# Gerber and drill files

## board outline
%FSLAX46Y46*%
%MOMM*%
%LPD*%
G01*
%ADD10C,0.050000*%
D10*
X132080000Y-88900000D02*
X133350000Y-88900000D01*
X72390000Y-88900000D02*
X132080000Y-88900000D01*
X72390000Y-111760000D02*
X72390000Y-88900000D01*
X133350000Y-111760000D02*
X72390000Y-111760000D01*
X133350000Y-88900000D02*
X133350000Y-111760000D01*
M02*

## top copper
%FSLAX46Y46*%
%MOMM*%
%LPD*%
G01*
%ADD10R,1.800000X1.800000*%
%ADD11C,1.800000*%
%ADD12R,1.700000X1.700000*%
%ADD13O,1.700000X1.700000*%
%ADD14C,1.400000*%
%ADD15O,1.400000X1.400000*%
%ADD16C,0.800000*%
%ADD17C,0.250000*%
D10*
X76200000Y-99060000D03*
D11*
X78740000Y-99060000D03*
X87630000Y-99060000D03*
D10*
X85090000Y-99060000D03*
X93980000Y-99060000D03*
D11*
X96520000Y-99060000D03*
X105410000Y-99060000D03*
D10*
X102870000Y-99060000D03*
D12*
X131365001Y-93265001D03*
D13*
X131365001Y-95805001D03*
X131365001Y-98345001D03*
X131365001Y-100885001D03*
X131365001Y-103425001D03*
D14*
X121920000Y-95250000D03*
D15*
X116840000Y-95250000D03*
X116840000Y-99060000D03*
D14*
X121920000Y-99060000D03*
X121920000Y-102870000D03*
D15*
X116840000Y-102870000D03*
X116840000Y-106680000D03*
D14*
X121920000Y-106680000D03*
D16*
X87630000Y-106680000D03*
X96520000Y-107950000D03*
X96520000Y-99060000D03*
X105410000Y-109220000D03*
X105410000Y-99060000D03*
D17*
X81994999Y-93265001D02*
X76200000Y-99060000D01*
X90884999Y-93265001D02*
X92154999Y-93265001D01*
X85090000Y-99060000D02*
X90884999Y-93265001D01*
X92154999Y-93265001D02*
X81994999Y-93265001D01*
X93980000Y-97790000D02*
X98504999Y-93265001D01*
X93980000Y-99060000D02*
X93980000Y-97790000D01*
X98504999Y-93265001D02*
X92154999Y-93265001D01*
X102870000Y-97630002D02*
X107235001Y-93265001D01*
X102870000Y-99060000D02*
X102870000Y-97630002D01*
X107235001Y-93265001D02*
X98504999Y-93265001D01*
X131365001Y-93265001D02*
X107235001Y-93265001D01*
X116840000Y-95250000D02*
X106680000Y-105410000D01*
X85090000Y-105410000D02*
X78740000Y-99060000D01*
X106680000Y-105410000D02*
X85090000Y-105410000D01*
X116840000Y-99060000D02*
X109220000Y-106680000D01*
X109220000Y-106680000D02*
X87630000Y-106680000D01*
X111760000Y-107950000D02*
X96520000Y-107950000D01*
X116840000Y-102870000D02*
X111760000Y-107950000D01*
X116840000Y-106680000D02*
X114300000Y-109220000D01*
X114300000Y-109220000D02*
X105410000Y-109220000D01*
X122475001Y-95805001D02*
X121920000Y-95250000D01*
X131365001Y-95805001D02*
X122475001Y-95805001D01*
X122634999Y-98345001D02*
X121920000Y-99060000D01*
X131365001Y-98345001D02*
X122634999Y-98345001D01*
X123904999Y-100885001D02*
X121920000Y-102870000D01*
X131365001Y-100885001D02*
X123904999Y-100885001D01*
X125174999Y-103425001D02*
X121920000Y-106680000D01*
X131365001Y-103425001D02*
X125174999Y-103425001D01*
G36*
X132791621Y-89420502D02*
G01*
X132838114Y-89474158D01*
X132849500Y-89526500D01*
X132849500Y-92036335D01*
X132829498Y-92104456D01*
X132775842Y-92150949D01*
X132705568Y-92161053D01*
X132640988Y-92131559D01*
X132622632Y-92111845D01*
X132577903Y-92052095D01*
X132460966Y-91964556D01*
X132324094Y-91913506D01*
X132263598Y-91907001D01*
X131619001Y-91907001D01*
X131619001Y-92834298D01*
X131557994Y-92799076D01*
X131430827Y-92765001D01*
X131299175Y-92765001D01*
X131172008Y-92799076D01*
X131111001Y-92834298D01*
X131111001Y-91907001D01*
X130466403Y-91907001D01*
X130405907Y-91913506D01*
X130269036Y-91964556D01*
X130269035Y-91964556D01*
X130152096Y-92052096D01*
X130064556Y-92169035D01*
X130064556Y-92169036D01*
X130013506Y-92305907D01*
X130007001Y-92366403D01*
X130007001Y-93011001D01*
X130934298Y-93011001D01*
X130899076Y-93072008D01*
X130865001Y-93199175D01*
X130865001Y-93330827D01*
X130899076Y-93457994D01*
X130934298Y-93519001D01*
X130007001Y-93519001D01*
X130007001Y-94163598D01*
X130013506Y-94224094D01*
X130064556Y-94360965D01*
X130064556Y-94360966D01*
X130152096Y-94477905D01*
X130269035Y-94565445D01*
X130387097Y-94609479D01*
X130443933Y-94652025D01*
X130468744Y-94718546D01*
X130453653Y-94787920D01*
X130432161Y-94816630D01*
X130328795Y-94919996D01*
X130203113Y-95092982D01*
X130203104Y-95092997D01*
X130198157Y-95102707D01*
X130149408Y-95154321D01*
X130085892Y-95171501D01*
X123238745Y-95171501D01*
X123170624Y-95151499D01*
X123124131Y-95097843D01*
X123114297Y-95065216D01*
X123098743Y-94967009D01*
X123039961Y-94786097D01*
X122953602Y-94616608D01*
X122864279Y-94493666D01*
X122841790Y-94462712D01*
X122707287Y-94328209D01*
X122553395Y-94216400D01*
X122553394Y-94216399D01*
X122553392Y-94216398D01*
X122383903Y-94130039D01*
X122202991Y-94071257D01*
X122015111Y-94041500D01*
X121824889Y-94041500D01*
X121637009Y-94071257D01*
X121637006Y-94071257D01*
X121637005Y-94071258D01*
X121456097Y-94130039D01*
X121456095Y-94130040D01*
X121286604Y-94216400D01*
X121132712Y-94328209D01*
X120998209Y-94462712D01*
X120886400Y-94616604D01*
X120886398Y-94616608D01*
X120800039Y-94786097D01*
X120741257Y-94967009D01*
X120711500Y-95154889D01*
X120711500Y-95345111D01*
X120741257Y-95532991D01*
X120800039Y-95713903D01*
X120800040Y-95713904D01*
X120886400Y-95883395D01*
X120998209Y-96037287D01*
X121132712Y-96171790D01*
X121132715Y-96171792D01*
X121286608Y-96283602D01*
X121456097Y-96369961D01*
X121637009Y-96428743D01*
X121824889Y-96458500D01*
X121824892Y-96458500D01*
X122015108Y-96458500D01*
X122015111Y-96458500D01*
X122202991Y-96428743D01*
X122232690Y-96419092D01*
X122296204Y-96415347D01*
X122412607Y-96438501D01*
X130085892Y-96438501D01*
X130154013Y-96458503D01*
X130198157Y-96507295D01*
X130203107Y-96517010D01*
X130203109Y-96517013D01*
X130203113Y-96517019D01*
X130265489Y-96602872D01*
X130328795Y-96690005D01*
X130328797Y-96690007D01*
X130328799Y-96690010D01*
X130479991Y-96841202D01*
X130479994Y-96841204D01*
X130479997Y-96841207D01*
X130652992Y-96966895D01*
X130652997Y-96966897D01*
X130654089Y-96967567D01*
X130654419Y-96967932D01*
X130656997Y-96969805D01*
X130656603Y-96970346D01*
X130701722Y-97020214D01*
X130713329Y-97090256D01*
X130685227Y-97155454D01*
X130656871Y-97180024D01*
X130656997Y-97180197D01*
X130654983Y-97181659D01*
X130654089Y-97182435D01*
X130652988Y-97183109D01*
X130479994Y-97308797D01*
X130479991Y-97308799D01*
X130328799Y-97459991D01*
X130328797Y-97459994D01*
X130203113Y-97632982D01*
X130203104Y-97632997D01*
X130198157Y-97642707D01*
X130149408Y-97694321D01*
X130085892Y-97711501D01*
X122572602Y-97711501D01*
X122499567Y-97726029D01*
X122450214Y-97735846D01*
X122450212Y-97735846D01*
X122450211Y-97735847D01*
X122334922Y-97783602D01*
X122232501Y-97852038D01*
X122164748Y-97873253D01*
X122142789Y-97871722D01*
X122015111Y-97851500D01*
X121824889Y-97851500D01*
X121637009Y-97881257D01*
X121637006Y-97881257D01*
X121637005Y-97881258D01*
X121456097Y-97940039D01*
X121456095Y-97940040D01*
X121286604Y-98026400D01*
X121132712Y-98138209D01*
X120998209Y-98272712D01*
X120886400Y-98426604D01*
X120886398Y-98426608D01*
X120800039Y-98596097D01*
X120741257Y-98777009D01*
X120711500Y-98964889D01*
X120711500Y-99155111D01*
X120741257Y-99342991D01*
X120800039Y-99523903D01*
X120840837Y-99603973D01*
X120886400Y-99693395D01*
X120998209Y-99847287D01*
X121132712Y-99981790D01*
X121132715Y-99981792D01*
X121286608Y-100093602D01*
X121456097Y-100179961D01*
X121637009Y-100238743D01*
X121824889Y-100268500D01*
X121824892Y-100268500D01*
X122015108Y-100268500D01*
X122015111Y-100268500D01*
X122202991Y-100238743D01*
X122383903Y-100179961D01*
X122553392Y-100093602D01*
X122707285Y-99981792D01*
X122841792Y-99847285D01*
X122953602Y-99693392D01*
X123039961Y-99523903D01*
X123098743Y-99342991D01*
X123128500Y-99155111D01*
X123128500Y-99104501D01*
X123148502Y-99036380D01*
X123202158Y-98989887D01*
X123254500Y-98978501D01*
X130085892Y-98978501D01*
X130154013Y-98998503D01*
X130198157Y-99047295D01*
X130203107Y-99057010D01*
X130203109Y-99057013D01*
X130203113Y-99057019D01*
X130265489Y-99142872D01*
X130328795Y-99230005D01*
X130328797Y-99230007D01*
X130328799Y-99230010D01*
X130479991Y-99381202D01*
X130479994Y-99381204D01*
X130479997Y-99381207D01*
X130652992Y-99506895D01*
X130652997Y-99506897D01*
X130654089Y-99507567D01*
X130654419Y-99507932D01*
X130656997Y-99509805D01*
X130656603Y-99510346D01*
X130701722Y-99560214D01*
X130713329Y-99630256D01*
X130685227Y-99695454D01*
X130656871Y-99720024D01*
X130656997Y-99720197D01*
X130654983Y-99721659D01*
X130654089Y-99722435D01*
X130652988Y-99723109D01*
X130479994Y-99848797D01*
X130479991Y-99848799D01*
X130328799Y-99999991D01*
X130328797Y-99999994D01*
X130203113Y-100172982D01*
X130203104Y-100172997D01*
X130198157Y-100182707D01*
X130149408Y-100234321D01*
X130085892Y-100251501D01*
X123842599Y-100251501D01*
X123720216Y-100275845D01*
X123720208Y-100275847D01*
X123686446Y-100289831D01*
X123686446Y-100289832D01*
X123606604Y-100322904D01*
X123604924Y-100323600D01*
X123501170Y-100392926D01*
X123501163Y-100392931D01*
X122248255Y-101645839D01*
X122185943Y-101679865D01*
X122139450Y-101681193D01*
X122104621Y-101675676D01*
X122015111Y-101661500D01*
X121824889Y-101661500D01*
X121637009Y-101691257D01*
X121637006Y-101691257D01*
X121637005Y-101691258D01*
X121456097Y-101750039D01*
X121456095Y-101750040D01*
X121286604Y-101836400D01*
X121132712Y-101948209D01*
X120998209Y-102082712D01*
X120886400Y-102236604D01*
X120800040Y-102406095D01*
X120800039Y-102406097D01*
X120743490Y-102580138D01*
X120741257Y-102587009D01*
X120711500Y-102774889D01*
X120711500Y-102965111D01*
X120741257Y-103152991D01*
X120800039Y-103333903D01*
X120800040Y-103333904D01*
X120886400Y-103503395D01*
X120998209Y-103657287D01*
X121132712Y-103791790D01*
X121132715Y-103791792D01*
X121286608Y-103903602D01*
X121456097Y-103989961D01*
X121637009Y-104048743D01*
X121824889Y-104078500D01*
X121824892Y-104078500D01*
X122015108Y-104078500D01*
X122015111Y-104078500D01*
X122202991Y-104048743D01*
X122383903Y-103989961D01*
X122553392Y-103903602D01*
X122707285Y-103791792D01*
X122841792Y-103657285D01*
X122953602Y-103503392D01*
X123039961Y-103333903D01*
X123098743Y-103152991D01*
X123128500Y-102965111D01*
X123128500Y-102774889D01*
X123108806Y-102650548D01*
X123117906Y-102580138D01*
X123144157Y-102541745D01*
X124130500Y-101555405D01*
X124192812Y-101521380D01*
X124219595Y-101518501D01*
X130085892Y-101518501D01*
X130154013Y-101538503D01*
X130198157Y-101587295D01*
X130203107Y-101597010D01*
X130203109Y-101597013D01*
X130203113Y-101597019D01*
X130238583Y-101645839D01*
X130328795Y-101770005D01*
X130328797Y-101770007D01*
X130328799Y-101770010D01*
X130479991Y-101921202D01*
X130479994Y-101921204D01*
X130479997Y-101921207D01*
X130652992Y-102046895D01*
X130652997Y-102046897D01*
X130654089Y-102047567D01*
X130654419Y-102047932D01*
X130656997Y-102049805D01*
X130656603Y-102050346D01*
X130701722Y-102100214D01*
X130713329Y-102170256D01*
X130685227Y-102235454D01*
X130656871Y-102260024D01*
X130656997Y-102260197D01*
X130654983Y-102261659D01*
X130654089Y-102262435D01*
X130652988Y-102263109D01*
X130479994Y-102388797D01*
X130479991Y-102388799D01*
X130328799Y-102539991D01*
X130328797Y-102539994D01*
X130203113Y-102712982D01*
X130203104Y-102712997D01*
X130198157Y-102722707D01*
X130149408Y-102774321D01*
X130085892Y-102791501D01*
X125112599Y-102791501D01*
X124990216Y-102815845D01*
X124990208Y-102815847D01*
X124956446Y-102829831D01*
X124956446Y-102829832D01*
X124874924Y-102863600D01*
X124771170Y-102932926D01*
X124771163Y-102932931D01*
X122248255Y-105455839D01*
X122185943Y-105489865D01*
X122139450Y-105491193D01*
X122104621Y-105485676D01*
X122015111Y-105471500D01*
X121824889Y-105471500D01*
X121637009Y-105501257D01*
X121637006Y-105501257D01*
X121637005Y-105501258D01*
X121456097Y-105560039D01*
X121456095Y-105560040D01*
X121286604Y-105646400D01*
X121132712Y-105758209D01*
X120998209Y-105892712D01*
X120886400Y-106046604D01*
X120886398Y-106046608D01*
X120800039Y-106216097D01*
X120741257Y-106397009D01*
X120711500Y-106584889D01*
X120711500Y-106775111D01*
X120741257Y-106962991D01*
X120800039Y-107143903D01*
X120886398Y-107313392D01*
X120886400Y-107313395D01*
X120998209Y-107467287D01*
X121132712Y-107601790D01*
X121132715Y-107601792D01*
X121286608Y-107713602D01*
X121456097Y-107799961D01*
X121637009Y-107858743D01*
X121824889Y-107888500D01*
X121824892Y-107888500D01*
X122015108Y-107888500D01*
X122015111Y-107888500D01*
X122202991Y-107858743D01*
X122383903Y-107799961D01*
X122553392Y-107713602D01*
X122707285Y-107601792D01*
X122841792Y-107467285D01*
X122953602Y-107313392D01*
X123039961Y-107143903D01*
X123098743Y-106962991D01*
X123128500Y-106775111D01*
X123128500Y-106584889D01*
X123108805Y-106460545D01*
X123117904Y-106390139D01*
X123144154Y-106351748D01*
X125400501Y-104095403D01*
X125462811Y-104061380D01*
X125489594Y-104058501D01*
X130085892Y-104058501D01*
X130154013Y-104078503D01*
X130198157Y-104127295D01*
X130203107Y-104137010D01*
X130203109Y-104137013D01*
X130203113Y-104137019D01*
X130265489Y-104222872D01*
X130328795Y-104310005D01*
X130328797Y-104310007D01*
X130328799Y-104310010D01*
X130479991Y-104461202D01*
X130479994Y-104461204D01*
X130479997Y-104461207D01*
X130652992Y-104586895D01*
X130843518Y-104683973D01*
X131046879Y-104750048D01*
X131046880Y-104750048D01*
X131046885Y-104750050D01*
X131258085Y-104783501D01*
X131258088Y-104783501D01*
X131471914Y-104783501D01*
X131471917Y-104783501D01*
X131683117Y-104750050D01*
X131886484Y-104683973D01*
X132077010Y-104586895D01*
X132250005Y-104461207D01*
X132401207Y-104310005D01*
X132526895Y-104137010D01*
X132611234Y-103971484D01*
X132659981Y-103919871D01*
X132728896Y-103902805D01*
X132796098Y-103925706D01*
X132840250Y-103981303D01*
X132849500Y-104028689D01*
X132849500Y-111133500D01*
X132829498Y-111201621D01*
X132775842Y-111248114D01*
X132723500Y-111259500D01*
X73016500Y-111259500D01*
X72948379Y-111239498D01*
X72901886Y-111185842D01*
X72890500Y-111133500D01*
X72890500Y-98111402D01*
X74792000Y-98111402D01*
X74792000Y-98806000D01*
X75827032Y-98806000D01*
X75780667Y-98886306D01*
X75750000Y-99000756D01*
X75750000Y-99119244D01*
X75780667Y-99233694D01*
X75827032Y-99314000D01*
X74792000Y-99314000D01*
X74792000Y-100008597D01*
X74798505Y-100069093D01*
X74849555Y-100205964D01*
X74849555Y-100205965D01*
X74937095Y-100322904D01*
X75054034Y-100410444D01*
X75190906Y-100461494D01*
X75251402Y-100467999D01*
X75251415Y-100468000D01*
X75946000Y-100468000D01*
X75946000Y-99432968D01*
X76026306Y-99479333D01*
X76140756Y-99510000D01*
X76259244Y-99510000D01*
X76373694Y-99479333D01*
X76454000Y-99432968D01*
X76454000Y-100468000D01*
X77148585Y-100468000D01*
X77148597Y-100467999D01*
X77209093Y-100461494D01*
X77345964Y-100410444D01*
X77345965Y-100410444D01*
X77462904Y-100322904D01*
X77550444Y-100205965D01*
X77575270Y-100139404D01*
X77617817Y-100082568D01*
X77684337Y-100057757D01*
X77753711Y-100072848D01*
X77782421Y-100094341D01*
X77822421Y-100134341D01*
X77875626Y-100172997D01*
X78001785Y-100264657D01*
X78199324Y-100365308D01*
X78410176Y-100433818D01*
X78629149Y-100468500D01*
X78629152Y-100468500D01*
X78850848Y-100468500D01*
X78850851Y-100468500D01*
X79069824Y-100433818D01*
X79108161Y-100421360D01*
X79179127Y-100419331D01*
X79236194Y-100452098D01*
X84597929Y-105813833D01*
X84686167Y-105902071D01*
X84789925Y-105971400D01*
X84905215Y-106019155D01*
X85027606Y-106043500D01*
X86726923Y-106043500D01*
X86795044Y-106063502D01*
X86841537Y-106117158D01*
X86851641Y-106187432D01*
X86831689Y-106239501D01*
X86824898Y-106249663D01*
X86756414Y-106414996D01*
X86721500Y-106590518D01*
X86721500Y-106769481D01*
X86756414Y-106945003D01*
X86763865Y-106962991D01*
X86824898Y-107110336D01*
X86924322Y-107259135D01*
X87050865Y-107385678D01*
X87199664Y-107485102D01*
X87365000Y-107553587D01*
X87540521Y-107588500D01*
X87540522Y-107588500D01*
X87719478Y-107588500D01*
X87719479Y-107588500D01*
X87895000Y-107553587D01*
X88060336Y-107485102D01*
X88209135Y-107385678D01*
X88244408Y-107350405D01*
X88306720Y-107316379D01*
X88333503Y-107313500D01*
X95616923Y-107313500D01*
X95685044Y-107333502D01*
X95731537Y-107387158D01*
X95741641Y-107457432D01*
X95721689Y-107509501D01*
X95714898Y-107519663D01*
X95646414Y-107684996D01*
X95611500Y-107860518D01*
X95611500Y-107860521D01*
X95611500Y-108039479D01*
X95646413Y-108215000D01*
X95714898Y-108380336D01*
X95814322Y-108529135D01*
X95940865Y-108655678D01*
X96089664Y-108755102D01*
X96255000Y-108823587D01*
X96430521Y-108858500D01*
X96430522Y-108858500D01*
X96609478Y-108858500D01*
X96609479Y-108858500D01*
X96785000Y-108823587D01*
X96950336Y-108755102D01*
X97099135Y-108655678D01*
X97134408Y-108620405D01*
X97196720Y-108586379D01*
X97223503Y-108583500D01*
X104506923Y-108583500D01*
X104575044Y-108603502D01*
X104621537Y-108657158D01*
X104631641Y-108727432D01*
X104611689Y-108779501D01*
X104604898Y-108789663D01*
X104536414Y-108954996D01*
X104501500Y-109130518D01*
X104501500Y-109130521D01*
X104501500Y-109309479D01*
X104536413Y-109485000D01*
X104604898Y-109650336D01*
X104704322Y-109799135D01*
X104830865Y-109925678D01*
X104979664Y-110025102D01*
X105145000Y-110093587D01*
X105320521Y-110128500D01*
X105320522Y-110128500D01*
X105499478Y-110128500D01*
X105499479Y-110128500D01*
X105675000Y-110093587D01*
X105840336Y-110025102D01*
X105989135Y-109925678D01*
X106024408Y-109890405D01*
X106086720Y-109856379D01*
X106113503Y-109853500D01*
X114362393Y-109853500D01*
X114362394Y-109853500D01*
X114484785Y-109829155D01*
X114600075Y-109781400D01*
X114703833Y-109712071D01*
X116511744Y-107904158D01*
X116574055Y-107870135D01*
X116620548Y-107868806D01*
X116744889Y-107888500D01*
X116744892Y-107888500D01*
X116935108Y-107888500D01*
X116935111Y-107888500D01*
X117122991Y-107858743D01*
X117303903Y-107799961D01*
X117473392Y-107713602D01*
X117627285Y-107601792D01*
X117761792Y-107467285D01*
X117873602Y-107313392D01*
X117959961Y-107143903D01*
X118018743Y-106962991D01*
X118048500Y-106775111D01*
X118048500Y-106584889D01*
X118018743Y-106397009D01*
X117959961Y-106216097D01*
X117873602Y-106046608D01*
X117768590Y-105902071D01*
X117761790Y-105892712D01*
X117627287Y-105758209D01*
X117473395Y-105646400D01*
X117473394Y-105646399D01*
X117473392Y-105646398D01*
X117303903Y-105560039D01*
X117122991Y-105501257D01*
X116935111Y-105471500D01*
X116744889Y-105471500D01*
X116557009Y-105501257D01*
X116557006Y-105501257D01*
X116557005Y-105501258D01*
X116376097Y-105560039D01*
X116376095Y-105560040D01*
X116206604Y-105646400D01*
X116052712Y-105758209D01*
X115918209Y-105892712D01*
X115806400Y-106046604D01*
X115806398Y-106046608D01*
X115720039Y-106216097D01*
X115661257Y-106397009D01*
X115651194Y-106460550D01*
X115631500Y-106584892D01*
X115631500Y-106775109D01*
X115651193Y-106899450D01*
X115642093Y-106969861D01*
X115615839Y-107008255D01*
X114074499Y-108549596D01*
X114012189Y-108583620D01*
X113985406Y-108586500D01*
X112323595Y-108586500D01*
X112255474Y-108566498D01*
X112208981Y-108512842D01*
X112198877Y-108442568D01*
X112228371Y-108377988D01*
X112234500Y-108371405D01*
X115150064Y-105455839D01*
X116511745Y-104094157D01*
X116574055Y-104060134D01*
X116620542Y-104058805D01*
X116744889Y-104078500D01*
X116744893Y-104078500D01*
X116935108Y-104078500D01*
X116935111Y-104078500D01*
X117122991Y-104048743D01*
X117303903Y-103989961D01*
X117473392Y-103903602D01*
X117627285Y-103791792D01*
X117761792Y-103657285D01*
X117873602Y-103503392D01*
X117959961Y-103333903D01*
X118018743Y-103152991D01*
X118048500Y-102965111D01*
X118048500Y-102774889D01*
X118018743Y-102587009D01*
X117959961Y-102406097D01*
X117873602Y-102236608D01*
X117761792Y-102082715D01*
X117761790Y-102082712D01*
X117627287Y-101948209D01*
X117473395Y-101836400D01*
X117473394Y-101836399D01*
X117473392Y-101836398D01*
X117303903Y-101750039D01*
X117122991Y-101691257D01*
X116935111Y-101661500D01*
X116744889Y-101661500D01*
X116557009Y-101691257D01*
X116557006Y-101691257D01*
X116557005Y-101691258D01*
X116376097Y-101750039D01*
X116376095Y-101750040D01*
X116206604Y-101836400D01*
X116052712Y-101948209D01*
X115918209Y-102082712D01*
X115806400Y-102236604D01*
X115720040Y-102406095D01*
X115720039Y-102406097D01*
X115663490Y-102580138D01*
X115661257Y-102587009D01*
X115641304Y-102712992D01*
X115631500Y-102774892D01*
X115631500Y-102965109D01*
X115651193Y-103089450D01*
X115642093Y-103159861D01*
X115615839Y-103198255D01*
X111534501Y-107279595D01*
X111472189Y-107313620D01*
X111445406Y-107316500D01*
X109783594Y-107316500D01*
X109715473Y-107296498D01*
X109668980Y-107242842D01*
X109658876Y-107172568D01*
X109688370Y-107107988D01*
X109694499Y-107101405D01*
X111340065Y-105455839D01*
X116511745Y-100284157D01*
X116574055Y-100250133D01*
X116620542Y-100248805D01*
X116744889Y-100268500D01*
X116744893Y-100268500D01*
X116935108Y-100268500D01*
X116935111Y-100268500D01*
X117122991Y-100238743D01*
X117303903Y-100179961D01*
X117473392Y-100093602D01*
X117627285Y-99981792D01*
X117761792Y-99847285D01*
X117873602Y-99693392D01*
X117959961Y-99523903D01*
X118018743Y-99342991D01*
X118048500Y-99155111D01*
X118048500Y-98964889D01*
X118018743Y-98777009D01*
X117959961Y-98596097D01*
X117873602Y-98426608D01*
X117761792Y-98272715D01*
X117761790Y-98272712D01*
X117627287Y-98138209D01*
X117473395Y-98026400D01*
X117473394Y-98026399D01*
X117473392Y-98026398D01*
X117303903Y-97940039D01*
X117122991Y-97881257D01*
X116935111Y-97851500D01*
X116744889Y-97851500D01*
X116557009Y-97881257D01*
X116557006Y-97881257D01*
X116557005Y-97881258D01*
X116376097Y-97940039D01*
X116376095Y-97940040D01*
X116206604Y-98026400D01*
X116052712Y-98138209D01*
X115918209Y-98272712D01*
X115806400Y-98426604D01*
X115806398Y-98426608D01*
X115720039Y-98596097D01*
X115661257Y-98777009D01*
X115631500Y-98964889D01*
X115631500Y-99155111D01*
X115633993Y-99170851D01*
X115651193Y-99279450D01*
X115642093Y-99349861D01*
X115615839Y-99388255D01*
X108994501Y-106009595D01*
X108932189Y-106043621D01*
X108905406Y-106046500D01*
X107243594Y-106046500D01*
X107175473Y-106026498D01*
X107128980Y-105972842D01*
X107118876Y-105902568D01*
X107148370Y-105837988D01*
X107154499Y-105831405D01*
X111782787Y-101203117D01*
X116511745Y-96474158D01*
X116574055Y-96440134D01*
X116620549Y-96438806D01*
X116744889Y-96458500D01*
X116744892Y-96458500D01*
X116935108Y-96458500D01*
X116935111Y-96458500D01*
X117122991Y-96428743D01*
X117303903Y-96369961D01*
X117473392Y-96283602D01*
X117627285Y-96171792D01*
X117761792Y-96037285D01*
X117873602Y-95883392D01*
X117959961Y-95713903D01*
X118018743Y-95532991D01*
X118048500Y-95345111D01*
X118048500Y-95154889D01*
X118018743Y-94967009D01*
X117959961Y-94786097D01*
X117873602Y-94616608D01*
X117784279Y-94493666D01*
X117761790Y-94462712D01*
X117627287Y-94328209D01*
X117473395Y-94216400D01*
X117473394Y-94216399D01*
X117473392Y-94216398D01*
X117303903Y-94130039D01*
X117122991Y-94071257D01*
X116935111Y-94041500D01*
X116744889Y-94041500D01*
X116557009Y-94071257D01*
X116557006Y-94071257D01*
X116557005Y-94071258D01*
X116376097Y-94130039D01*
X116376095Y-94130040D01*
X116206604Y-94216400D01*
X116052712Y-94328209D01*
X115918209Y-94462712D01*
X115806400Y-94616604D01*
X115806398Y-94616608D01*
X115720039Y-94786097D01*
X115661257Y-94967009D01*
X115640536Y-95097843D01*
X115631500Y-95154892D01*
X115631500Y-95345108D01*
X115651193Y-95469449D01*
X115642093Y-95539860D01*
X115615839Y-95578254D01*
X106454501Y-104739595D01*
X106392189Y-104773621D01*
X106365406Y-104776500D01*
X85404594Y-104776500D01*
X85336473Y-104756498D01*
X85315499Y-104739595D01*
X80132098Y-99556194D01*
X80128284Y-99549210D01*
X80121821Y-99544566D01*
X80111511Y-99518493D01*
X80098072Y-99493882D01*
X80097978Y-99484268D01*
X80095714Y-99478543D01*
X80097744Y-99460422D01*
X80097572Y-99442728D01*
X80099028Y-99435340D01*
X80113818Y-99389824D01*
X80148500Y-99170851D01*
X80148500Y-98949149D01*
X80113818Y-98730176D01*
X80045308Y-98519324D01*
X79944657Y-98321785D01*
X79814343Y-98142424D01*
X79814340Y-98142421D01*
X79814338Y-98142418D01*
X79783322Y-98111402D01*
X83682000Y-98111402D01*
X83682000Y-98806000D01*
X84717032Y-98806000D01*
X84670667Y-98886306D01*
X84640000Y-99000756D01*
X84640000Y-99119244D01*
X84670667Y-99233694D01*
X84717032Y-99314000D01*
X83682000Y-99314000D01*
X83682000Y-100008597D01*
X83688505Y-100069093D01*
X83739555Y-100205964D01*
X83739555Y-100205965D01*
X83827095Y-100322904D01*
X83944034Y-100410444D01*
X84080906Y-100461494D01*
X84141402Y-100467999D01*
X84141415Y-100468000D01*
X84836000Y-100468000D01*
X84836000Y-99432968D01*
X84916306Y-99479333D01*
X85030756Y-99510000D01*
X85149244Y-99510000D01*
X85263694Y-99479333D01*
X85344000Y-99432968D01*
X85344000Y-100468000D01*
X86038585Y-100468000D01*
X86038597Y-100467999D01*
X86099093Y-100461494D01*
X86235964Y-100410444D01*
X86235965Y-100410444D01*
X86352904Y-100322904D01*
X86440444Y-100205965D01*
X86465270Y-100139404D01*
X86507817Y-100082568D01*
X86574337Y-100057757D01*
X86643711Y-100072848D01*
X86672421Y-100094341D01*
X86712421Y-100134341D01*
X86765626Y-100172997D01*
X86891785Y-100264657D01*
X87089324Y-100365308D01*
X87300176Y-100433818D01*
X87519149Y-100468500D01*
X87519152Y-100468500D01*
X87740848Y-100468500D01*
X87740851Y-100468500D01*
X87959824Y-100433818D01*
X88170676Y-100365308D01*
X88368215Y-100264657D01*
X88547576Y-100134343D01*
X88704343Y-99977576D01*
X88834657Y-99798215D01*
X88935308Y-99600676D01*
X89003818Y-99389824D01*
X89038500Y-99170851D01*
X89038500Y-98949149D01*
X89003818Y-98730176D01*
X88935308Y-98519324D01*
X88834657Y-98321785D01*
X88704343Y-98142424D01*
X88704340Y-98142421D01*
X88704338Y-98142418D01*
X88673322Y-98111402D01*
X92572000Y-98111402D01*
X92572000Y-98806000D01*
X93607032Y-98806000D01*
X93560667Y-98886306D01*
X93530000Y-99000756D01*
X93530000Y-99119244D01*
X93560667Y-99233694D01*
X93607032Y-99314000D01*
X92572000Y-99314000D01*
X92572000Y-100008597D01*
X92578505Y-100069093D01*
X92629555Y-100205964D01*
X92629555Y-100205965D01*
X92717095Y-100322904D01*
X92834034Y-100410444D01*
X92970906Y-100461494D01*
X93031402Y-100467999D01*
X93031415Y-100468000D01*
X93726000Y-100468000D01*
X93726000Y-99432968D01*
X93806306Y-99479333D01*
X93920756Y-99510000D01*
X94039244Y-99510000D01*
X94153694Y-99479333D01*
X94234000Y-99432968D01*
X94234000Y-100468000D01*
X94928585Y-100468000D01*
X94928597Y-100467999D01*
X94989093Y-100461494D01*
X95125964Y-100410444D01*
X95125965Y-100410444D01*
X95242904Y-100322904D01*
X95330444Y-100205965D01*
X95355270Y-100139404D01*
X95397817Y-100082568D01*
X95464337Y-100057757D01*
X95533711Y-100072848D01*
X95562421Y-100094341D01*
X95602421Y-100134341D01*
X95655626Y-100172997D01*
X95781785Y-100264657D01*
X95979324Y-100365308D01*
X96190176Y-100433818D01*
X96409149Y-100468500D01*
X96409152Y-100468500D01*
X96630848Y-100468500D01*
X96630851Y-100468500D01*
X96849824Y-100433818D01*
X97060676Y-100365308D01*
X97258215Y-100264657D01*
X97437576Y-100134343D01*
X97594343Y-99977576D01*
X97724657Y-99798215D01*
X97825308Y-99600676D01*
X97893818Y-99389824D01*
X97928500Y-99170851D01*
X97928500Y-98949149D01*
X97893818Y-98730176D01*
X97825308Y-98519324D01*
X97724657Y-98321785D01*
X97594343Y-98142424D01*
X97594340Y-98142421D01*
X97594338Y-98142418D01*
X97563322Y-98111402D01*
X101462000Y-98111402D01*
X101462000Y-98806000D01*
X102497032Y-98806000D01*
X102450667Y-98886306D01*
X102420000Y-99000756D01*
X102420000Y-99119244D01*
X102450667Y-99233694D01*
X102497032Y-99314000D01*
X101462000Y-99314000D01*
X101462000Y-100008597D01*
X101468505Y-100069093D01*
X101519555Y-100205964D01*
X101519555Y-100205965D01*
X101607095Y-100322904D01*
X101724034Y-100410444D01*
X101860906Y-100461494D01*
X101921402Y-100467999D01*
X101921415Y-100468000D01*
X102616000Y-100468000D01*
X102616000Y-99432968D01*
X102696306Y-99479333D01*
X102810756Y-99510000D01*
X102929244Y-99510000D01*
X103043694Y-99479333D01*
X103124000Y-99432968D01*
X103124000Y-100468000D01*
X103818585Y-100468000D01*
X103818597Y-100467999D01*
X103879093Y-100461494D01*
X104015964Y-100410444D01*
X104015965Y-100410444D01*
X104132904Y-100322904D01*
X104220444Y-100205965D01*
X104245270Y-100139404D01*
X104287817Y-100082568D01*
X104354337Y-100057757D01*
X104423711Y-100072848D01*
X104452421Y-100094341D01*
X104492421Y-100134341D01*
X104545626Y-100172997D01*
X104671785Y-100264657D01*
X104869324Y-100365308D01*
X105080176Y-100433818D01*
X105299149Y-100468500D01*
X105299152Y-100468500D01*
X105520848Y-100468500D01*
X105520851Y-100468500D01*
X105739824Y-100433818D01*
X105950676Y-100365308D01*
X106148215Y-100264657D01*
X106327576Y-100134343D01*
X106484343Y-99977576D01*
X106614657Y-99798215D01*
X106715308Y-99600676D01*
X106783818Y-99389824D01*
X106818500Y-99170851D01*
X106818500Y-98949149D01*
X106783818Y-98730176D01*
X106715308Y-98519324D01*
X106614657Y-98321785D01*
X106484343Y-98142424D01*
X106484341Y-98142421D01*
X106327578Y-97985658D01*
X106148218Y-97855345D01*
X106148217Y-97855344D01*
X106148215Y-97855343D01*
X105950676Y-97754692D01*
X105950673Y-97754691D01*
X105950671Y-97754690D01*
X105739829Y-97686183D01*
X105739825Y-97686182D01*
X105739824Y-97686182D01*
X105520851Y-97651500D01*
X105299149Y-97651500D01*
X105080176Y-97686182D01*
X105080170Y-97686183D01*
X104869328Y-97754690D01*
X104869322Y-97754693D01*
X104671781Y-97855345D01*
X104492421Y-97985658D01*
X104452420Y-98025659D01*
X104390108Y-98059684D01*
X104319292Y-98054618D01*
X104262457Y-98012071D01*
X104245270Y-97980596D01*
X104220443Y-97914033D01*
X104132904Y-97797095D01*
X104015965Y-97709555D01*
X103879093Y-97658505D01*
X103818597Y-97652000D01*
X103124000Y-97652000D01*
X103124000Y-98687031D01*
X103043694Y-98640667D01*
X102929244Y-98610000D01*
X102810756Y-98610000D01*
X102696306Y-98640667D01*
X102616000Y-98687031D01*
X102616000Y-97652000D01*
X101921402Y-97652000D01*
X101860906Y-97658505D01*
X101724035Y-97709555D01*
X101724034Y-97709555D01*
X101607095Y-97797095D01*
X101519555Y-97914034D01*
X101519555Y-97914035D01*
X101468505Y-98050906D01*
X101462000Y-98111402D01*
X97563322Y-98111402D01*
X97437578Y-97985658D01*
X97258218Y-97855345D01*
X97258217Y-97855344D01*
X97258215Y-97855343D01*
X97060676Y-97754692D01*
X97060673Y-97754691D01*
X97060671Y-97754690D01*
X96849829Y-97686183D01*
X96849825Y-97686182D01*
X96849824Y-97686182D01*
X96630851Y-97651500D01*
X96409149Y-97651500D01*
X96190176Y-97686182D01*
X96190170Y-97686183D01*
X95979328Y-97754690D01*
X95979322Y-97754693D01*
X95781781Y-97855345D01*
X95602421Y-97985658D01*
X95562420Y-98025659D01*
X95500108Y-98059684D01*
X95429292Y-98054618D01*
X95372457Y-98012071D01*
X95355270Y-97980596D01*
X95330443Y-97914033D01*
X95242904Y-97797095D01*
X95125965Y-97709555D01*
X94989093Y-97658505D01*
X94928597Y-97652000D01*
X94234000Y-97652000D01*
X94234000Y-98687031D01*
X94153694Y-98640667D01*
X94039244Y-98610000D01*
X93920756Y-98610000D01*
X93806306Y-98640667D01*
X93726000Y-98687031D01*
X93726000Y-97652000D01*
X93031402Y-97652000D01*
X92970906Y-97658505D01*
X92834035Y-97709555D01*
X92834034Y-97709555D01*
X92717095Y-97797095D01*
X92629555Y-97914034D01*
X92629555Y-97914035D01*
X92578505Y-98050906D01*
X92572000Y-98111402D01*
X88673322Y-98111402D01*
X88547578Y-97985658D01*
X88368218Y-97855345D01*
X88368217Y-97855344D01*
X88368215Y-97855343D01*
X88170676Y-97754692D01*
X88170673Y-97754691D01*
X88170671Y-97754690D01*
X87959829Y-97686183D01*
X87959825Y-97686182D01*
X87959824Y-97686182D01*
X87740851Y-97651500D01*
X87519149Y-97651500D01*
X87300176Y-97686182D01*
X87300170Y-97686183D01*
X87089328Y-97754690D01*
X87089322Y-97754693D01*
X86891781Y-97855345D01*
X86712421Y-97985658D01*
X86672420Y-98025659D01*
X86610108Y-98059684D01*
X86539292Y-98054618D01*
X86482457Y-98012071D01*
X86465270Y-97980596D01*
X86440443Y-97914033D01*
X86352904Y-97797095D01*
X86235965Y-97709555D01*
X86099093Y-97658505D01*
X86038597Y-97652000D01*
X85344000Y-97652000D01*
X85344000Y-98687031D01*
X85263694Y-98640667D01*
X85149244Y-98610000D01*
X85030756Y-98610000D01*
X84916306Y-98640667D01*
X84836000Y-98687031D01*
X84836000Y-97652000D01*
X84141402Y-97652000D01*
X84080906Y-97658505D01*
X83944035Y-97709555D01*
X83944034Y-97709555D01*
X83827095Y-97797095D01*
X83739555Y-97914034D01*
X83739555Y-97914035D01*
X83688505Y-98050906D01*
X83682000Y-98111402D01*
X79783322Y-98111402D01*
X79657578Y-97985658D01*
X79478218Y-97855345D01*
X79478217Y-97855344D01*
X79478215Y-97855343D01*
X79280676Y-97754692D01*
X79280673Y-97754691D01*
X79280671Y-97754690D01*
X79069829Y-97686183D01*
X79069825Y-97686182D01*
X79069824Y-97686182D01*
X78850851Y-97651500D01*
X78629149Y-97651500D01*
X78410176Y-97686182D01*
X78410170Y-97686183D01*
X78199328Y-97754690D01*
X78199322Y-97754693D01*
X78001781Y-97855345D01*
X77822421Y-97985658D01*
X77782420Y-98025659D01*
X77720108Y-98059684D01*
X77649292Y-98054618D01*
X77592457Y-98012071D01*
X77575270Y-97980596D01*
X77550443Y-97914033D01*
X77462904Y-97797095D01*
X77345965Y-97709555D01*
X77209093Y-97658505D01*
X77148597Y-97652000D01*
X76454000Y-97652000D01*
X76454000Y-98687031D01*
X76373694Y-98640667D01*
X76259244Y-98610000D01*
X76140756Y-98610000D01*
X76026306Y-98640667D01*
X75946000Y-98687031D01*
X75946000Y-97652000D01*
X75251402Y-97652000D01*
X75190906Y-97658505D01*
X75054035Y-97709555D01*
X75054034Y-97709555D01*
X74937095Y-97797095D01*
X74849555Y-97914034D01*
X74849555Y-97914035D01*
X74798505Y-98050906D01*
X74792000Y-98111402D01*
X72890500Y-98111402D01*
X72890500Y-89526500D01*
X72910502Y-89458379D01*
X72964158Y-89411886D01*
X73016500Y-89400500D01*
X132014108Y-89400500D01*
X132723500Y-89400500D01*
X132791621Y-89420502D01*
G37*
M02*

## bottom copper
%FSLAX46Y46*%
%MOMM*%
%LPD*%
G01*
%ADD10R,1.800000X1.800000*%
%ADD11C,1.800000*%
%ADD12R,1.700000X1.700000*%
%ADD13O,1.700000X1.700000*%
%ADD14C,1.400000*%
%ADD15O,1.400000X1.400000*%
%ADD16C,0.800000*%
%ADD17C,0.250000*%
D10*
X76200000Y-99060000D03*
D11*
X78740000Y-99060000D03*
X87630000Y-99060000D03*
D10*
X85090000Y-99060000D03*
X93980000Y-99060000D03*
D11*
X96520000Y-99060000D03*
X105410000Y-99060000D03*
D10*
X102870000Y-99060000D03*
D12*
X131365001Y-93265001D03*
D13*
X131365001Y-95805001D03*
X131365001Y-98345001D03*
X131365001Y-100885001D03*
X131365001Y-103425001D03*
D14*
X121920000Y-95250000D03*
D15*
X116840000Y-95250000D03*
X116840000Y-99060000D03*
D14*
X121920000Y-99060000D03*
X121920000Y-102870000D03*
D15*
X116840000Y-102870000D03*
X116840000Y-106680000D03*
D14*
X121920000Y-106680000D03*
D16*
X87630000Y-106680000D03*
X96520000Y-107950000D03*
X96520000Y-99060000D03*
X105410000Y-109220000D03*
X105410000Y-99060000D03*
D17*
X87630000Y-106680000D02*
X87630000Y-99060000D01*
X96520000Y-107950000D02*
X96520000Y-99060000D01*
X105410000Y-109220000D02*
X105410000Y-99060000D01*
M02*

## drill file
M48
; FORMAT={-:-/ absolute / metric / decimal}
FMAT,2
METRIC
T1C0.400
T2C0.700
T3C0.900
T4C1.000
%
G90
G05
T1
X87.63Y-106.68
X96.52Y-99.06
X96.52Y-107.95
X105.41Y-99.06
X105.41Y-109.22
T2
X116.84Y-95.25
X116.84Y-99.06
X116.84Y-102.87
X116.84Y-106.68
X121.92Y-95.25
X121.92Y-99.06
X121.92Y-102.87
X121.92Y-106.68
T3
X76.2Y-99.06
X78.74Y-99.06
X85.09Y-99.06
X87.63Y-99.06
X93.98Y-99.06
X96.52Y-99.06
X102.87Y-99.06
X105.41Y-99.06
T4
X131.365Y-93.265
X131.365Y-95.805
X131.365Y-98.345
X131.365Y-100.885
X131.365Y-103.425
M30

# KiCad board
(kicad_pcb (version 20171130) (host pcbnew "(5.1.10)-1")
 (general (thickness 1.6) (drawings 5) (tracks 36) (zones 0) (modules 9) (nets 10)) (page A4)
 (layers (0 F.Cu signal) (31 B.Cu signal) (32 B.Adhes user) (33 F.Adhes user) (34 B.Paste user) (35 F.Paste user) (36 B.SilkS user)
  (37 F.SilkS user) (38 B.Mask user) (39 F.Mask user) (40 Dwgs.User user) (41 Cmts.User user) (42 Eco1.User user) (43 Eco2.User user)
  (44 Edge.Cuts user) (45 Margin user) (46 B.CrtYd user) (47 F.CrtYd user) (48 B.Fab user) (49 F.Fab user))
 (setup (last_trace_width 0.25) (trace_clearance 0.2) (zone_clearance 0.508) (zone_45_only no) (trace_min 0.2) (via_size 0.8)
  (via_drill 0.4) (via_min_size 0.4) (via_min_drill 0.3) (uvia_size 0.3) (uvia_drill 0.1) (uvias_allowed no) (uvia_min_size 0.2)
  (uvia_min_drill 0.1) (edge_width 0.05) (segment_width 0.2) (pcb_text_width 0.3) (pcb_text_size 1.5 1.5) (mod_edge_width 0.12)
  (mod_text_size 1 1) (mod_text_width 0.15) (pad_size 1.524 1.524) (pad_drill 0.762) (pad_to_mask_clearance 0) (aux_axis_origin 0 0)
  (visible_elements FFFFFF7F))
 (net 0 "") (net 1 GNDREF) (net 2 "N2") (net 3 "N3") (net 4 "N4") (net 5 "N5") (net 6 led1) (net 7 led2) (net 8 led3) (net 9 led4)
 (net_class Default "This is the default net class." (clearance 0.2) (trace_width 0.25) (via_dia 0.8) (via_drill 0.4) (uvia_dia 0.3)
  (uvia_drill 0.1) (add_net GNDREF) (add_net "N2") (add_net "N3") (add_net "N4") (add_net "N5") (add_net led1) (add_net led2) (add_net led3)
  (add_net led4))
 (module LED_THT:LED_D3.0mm (layer F.Cu) (at 76.2 99.06)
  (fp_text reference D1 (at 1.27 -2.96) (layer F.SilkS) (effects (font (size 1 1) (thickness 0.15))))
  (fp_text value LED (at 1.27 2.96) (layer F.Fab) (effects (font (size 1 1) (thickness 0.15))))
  (pad 1 thru_hole rect (at 0 0) (size 1.8 1.8) (drill 0.9) (layers *.Cu *.Mask) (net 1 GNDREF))
  (pad 2 thru_hole circle (at 2.54 0) (size 1.8 1.8) (drill 0.9) (layers *.Cu *.Mask) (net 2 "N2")))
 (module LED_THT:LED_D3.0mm (layer F.Cu) (at 85.09 99.06)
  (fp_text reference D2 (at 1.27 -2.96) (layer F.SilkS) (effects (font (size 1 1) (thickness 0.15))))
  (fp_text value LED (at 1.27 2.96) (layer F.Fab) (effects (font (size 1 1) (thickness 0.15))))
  (pad 2 thru_hole circle (at 2.54 0) (size 1.8 1.8) (drill 0.9) (layers *.Cu *.Mask) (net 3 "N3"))
  (pad 1 thru_hole rect (at 0 0) (size 1.8 1.8) (drill 0.9) (layers *.Cu *.Mask) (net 1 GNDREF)))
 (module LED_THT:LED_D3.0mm (layer F.Cu) (at 93.98 99.06)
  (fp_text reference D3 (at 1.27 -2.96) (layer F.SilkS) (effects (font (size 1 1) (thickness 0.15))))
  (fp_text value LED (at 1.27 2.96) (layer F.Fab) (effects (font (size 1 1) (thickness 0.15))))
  (pad 1 thru_hole rect (at 0 0) (size 1.8 1.8) (drill 0.9) (layers *.Cu *.Mask) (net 1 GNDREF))
  (pad 2 thru_hole circle (at 2.54 0) (size 1.8 1.8) (drill 0.9) (layers *.Cu *.Mask) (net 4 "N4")))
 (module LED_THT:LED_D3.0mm (layer F.Cu) (at 102.87 99.06)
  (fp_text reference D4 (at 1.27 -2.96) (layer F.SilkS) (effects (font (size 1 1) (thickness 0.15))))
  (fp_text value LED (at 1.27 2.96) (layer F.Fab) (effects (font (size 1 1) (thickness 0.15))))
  (pad 2 thru_hole circle (at 2.54 0) (size 1.8 1.8) (drill 0.9) (layers *.Cu *.Mask) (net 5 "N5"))
  (pad 1 thru_hole rect (at 0 0) (size 1.8 1.8) (drill 0.9) (layers *.Cu *.Mask) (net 1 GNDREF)))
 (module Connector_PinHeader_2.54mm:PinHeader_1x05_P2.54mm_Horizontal (layer F.Cu) (at 131.365001 93.265001)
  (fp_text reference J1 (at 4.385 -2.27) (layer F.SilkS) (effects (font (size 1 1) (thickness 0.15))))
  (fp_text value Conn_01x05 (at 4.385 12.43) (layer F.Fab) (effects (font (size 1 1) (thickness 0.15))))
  (pad 1 thru_hole rect (at 0 0) (size 1.7 1.7) (drill 1) (layers *.Cu *.Mask) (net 1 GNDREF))
  (pad 2 thru_hole oval (at 0 2.54) (size 1.7 1.7) (drill 1) (layers *.Cu *.Mask) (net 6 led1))
  (pad 3 thru_hole oval (at 0 5.08) (size 1.7 1.7) (drill 1) (layers *.Cu *.Mask) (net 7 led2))
  (pad 4 thru_hole oval (at 0 7.62) (size 1.7 1.7) (drill 1) (layers *.Cu *.Mask) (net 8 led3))
  (pad 5 thru_hole oval (at 0 10.16) (size 1.7 1.7) (drill 1) (layers *.Cu *.Mask) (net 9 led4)))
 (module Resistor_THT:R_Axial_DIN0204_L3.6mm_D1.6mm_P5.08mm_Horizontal (layer F.Cu) (at 121.92 95.25 180)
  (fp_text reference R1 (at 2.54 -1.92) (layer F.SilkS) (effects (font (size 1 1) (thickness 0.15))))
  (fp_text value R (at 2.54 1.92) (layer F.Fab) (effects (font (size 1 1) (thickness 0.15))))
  (pad 1 thru_hole circle (at 0 0 180) (size 1.4 1.4) (drill 0.7) (layers *.Cu *.Mask) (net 6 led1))
  (pad 2 thru_hole oval (at 5.08 0 180) (size 1.4 1.4) (drill 0.7) (layers *.Cu *.Mask) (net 2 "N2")))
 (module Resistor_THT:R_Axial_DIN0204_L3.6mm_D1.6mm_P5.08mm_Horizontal (layer F.Cu) (at 121.92 99.06 180)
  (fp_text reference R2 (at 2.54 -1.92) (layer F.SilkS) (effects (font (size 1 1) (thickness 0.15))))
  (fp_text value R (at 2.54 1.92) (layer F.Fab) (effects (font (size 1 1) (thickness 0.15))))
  (pad 2 thru_hole oval (at 5.08 0 180) (size 1.4 1.4) (drill 0.7) (layers *.Cu *.Mask) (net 3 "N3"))
  (pad 1 thru_hole circle (at 0 0 180) (size 1.4 1.4) (drill 0.7) (layers *.Cu *.Mask) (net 7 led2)))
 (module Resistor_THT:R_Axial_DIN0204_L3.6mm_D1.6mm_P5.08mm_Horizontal (layer F.Cu) (at 121.92 102.87 180)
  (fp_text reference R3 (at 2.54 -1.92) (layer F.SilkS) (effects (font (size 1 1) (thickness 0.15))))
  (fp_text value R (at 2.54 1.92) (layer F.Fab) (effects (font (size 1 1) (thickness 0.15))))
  (pad 1 thru_hole circle (at 0 0 180) (size 1.4 1.4) (drill 0.7) (layers *.Cu *.Mask) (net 8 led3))
  (pad 2 thru_hole oval (at 5.08 0 180) (size 1.4 1.4) (drill 0.7) (layers *.Cu *.Mask) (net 4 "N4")))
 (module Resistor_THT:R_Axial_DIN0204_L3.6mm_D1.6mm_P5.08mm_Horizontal (layer F.Cu) (at 121.92 106.68 180)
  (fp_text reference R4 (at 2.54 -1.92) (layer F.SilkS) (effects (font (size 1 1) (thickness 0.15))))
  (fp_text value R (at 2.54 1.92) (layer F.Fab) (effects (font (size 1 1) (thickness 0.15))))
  (pad 2 thru_hole oval (at 5.08 0 180) (size 1.4 1.4) (drill 0.7) (layers *.Cu *.Mask) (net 5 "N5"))
  (pad 1 thru_hole circle (at 0 0 180) (size 1.4 1.4) (drill 0.7) (layers *.Cu *.Mask) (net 9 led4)))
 (gr_line (start 132.08 88.9) (end 133.35 88.9) (layer Edge.Cuts) (width 0.05))
 (gr_line (start 72.39 88.9) (end 132.08 88.9) (layer Edge.Cuts) (width 0.05))
 (gr_line (start 72.39 111.76) (end 72.39 88.9) (layer Edge.Cuts) (width 0.05))
 (gr_line (start 133.35 111.76) (end 72.39 111.76) (layer Edge.Cuts) (width 0.05))
 (gr_line (start 133.35 88.9) (end 133.35 111.76) (layer Edge.Cuts) (width 0.05))
 (segment (start 81.994999 93.265001) (end 76.2 99.06) (width 0.25) (layer F.Cu) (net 1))
 (segment (start 90.884999 93.265001) (end 92.154999 93.265001) (width 0.25) (layer F.Cu) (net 1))
 (segment (start 85.09 99.06) (end 90.884999 93.265001) (width 0.25) (layer F.Cu) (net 1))
 (segment (start 92.154999 93.265001) (end 81.994999 93.265001) (width 0.25) (layer F.Cu) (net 1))
 (segment (start 93.98 97.79) (end 98.504999 93.265001) (width 0.25) (layer F.Cu) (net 1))
 (segment (start 93.98 99.06) (end 93.98 97.79) (width 0.25) (layer F.Cu) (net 1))
 (segment (start 98.504999 93.265001) (end 92.154999 93.265001) (width 0.25) (layer F.Cu) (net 1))
 (segment (start 102.87 97.630002) (end 107.235001 93.265001) (width 0.25) (layer F.Cu) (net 1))
 (segment (start 102.87 99.06) (end 102.87 97.630002) (width 0.25) (layer F.Cu) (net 1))
 (segment (start 107.235001 93.265001) (end 98.504999 93.265001) (width 0.25) (layer F.Cu) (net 1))
 (segment (start 131.365001 93.265001) (end 107.235001 93.265001) (width 0.25) (layer F.Cu) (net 1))
 (segment (start 116.84 95.25) (end 106.68 105.41) (width 0.25) (layer F.Cu) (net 2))
 (segment (start 85.09 105.41) (end 78.74 99.06) (width 0.25) (layer F.Cu) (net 2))
 (segment (start 106.68 105.41) (end 85.09 105.41) (width 0.25) (layer F.Cu) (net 2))
 (segment (start 116.84 99.06) (end 109.22 106.68) (width 0.25) (layer F.Cu) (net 3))
 (via (at 87.63 106.68) (size 0.8) (drill 0.4) (layers F.Cu B.Cu) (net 3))
 (segment (start 109.22 106.68) (end 87.63 106.68) (width 0.25) (layer F.Cu) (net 3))
 (segment (start 87.63 106.68) (end 87.63 99.06) (width 0.25) (layer B.Cu) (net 3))
 (via (at 96.52 107.95) (size 0.8) (drill 0.4) (layers F.Cu B.Cu) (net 4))
 (segment (start 111.76 107.95) (end 96.52 107.95) (width 0.25) (layer F.Cu) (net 4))
 (segment (start 116.84 102.87) (end 111.76 107.95) (width 0.25) (layer F.Cu) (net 4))
 (via (at 96.52 99.06) (size 0.8) (drill 0.4) (layers F.Cu B.Cu) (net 4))
 (segment (start 96.52 107.95) (end 96.52 99.06) (width 0.25) (layer B.Cu) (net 4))
 (segment (start 116.84 106.68) (end 114.3 109.22) (width 0.25) (layer F.Cu) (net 5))
 (via (at 105.41 109.22) (size 0.8) (drill 0.4) (layers F.Cu B.Cu) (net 5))
 (segment (start 114.3 109.22) (end 105.41 109.22) (width 0.25) (layer F.Cu) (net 5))
 (via (at 105.41 99.06) (size 0.8) (drill 0.4) (layers F.Cu B.Cu) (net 5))
 (segment (start 105.41 109.22) (end 105.41 99.06) (width 0.25) (layer B.Cu) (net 5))
 (segment (start 122.475001 95.805001) (end 121.92 95.25) (width 0.25) (layer F.Cu) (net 6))
 (segment (start 131.365001 95.805001) (end 122.475001 95.805001) (width 0.25) (layer F.Cu) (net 6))
 (segment (start 122.634999 98.345001) (end 121.92 99.06) (width 0.25) (layer F.Cu) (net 7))
 (segment (start 131.365001 98.345001) (end 122.634999 98.345001) (width 0.25) (layer F.Cu) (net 7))
 (segment (start 123.904999 100.885001) (end 121.92 102.87) (width 0.25) (layer F.Cu) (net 8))
 (segment (start 131.365001 100.885001) (end 123.904999 100.885001) (width 0.25) (layer F.Cu) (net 8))
 (segment (start 125.174999 103.425001) (end 121.92 106.68) (width 0.25) (layer F.Cu) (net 9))
 (segment (start 131.365001 103.425001) (end 125.174999 103.425001) (width 0.25) (layer F.Cu) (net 9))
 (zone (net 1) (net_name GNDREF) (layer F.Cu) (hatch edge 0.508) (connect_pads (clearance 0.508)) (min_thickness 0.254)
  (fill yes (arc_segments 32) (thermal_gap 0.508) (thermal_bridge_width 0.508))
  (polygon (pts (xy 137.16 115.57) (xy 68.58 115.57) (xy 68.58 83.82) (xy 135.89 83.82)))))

